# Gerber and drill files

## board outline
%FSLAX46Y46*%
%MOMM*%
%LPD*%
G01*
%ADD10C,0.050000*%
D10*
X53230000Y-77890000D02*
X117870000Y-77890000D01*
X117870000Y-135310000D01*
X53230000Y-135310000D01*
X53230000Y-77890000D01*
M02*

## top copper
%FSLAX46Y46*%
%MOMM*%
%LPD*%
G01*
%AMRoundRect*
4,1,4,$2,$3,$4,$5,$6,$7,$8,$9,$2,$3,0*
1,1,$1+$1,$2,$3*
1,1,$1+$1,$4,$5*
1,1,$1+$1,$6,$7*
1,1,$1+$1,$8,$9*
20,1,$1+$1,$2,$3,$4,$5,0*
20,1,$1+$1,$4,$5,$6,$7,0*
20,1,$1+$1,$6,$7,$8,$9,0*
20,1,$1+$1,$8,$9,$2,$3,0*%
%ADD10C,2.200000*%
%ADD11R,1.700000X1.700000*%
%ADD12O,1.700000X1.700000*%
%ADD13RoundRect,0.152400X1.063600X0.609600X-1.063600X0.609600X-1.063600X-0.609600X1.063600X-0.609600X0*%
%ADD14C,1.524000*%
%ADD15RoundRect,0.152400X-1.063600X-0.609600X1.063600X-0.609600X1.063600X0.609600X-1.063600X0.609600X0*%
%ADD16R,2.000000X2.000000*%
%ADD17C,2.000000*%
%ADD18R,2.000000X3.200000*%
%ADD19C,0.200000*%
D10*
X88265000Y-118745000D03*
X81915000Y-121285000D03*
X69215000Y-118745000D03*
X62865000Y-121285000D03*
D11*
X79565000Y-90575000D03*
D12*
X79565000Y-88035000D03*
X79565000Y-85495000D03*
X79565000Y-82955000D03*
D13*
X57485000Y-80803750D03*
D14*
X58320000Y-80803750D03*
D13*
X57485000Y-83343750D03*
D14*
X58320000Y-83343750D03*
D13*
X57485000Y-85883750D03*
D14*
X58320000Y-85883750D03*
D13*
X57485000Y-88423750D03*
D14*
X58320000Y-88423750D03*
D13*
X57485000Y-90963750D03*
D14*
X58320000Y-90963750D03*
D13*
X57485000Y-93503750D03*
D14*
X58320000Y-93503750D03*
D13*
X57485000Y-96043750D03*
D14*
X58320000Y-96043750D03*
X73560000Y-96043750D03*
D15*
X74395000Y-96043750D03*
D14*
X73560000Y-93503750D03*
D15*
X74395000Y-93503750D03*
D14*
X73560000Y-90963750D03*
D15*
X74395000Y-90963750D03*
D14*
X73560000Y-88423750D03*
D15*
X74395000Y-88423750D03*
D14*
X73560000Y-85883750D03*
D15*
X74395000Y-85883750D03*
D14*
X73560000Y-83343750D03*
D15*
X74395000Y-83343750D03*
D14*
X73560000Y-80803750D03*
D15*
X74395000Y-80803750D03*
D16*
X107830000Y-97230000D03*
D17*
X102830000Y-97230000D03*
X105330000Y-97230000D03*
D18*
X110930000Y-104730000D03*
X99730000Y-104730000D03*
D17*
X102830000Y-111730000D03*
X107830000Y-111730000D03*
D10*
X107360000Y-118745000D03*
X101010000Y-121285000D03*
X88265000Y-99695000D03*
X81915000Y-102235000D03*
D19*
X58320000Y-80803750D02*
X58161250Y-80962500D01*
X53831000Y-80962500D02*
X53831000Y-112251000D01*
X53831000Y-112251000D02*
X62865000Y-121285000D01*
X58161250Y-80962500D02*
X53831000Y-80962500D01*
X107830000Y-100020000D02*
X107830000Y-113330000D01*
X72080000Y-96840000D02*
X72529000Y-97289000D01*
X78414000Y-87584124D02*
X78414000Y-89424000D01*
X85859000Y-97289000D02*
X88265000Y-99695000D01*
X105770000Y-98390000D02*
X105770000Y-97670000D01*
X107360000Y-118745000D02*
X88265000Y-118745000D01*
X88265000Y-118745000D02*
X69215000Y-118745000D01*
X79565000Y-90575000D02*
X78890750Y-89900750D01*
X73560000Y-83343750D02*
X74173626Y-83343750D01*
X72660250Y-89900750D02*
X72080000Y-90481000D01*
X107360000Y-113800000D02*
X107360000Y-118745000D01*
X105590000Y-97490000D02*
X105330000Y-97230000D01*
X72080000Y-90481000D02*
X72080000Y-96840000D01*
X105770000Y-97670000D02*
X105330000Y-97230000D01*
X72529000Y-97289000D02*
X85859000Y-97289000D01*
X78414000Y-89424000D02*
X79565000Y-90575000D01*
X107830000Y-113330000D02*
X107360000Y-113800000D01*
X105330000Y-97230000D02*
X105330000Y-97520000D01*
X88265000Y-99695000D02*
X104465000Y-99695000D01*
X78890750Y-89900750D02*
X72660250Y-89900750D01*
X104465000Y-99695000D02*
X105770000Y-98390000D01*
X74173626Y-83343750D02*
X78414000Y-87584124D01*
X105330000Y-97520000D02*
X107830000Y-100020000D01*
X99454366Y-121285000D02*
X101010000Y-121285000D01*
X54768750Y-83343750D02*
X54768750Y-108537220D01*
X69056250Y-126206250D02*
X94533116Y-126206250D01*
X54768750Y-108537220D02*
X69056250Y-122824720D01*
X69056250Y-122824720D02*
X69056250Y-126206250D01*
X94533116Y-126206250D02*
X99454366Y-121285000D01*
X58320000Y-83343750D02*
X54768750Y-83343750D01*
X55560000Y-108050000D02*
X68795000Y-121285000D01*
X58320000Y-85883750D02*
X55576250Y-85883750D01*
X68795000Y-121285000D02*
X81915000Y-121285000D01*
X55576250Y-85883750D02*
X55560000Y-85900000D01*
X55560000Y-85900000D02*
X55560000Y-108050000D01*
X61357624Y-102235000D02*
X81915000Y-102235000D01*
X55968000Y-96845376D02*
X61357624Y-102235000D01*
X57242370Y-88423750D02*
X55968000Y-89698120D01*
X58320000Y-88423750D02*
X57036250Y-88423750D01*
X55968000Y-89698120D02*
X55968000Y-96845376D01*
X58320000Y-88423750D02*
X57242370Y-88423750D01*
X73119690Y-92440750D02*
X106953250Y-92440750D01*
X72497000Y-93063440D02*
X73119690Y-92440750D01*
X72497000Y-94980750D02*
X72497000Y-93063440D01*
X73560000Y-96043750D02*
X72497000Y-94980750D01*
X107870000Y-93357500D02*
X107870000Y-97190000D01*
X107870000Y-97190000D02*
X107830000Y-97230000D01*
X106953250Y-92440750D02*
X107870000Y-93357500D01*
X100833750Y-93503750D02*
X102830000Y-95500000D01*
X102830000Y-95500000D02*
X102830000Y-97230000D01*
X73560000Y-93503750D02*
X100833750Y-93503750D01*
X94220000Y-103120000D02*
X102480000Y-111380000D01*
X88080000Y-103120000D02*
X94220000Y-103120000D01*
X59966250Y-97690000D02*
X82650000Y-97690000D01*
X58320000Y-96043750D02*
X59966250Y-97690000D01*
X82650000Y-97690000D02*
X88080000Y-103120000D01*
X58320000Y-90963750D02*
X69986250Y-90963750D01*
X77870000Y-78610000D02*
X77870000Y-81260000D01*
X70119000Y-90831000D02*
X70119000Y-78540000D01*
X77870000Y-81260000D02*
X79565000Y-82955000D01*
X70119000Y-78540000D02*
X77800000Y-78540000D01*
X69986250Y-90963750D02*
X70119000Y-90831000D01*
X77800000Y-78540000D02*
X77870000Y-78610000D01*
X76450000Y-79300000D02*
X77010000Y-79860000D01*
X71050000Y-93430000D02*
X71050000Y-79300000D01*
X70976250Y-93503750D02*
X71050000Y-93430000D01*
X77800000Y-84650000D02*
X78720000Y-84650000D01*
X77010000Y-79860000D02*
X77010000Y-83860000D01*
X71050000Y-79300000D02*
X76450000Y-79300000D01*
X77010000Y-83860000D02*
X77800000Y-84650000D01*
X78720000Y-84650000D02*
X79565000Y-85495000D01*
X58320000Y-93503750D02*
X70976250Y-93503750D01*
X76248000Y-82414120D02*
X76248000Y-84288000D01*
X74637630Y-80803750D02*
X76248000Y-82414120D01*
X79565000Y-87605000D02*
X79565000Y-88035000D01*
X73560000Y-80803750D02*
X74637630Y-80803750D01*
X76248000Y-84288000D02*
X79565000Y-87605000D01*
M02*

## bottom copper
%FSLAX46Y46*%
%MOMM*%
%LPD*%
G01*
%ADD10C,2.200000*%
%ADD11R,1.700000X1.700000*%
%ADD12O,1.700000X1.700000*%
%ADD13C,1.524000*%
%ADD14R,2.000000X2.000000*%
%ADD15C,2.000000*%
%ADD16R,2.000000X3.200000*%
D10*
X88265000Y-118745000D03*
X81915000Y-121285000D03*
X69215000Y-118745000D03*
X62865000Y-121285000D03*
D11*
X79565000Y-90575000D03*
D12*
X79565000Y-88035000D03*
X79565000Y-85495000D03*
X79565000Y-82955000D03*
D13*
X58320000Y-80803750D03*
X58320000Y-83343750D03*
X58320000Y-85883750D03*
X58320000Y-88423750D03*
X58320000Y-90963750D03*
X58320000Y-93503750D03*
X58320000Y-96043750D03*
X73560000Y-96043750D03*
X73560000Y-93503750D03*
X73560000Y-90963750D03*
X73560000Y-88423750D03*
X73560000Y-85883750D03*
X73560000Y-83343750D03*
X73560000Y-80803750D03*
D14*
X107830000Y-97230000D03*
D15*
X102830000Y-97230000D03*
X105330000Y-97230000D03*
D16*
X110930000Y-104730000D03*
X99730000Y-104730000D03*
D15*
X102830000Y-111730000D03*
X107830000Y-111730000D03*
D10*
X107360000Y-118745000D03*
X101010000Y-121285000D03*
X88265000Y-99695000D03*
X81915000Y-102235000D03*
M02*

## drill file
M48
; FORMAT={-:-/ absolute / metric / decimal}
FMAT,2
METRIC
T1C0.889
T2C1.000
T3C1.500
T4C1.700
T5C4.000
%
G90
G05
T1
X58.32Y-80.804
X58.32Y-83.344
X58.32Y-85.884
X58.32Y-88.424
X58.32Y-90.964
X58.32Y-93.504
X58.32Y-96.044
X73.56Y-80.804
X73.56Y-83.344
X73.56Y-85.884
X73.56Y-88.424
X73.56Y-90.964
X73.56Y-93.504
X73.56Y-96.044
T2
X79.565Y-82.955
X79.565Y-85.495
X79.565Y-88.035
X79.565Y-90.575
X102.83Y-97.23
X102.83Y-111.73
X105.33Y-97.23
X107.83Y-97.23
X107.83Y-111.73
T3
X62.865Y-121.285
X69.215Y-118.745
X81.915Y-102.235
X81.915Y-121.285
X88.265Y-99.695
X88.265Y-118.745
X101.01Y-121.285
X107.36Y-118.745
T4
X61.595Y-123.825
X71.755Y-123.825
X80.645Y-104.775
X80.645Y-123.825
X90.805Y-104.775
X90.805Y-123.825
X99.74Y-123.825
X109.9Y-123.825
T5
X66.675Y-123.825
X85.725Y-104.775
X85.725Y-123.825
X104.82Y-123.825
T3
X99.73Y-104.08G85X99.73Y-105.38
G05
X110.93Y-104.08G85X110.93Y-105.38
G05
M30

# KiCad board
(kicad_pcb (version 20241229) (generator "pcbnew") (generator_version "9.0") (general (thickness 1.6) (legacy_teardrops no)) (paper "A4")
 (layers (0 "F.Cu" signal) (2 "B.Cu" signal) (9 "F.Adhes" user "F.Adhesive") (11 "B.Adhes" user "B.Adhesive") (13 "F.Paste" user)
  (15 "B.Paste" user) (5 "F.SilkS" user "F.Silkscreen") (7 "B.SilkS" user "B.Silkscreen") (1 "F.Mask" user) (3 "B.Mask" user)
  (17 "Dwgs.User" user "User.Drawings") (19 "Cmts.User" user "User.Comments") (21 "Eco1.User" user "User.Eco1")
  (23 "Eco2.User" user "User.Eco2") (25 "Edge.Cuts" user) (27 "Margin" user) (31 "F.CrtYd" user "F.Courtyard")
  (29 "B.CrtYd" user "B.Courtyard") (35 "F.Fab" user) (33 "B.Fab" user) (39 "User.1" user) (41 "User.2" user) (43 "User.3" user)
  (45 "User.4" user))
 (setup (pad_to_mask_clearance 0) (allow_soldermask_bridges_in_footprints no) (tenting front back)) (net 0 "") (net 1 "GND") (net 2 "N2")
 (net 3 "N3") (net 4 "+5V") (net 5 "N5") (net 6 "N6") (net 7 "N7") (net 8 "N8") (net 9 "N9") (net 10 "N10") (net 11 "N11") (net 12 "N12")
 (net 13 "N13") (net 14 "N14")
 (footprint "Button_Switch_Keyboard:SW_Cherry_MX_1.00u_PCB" (layer "F.Cu") (at 88.265 118.745)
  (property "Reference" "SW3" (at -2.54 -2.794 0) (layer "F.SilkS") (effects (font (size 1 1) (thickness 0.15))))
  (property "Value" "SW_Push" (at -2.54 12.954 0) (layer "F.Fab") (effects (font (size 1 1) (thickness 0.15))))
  (pad "" np_thru_hole circle (at -7.62 5.08) (size 1.7 1.7) (drill 1.7) (layers "*.Cu" "*.Mask"))
  (pad "" np_thru_hole circle (at -2.54 5.08) (size 4 4) (drill 4) (layers "*.Cu" "*.Mask"))
  (pad "" np_thru_hole circle (at 2.54 5.08) (size 1.7 1.7) (drill 1.7) (layers "*.Cu" "*.Mask"))
  (pad "1" thru_hole circle (at 0 0) (size 2.2 2.2) (drill 1.5) (layers "*.Cu" "*.Mask") (remove_unused_layers no) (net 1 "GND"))
  (pad "2" thru_hole circle (at -6.35 2.54) (size 2.2 2.2) (drill 1.5) (layers "*.Cu" "*.Mask") (remove_unused_layers no) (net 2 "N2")))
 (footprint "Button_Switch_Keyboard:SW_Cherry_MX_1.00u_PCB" (layer "F.Cu") (at 69.215 118.745)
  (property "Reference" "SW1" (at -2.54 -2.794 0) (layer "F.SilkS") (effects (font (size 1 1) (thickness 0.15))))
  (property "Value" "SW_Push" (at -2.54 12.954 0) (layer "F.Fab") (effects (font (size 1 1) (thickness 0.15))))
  (pad "" np_thru_hole circle (at -7.62 5.08) (size 1.7 1.7) (drill 1.7) (layers "*.Cu" "*.Mask"))
  (pad "" np_thru_hole circle (at -2.54 5.08) (size 4 4) (drill 4) (layers "*.Cu" "*.Mask"))
  (pad "" np_thru_hole circle (at 2.54 5.08) (size 1.7 1.7) (drill 1.7) (layers "*.Cu" "*.Mask"))
  (pad "1" thru_hole circle (at 0 0) (size 2.2 2.2) (drill 1.5) (layers "*.Cu" "*.Mask") (remove_unused_layers no) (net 1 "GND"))
  (pad "2" thru_hole circle (at -6.35 2.54) (size 2.2 2.2) (drill 1.5) (layers "*.Cu" "*.Mask") (remove_unused_layers no) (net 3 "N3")))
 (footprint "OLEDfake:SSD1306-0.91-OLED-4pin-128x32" (layer "F.Cu") (at 116.065 92.765 180)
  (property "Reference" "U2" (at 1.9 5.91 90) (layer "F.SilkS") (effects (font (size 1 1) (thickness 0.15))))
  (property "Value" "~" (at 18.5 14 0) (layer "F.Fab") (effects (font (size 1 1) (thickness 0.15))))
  (pad "1" thru_hole rect (at 36.5 2.19 180) (size 1.7 1.7) (drill 1) (layers "*.Cu" "*.Mask") (remove_unused_layers no) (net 1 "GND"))
  (pad "2" thru_hole oval (at 36.5 4.73 180) (size 1.7 1.7) (drill 1) (layers "*.Cu" "*.Mask") (remove_unused_layers no) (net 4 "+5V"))
  (pad "3" thru_hole oval (at 36.5 7.27 180) (size 1.7 1.7) (drill 1) (layers "*.Cu" "*.Mask") (remove_unused_layers no) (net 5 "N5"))
  (pad "4" thru_hole oval (at 36.5 9.81 180) (size 1.7 1.7) (drill 1) (layers "*.Cu" "*.Mask") (remove_unused_layers no) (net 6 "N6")))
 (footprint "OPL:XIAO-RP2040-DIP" (layer "F.Cu") (at 65.94 88.42375)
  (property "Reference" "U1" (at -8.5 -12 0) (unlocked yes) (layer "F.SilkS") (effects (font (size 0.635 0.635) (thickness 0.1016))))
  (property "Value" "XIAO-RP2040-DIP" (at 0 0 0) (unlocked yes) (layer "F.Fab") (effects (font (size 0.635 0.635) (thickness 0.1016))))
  (pad "1" smd roundrect (at -8.455 -7.62 180) (size 2.432 1.524) (layers "F.Cu" "F.Mask") (roundrect_rratio 0.1) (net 3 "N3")
   (thermal_bridge_angle 45))
  (pad "1" thru_hole circle (at -7.62 -7.62 180) (size 1.524 1.524) (drill 0.889) (layers "*.Cu" "*.Mask") (remove_unused_layers no)
   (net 3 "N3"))
  (pad "2" smd roundrect (at -8.455 -5.08 180) (size 2.432 1.524) (layers "F.Cu" "F.Mask") (roundrect_rratio 0.1) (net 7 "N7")
   (thermal_bridge_angle 45))
  (pad "2" thru_hole circle (at -7.62 -5.08 180) (size 1.524 1.524) (drill 0.889) (layers "*.Cu" "*.Mask") (remove_unused_layers no)
   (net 7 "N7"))
  (pad "3" smd roundrect (at -8.455 -2.54 180) (size 2.432 1.524) (layers "F.Cu" "F.Mask") (roundrect_rratio 0.1) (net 2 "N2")
   (thermal_bridge_angle 45))
  (pad "3" thru_hole circle (at -7.62 -2.54 180) (size 1.524 1.524) (drill 0.889) (layers "*.Cu" "*.Mask") (remove_unused_layers no)
   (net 2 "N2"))
  (pad "4" smd roundrect (at -8.455 0 180) (size 2.432 1.524) (layers "F.Cu" "F.Mask") (roundrect_rratio 0.1) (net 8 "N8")
   (thermal_bridge_angle 45))
  (pad "4" thru_hole circle (at -7.62 0 180) (size 1.524 1.524) (drill 0.889) (layers "*.Cu" "*.Mask") (remove_unused_layers no)
   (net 8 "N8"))
  (pad "5" smd roundrect (at -8.455 2.54 180) (size 2.432 1.524) (layers "F.Cu" "F.Mask") (roundrect_rratio 0.1) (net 6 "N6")
   (thermal_bridge_angle 45))
  (pad "5" thru_hole circle (at -7.62 2.54 180) (size 1.524 1.524) (drill 0.889) (layers "*.Cu" "*.Mask") (remove_unused_layers no)
   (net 6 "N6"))
  (pad "6" smd roundrect (at -8.455 5.08 180) (size 2.432 1.524) (layers "F.Cu" "F.Mask") (roundrect_rratio 0.1) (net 5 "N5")
   (thermal_bridge_angle 45))
  (pad "6" thru_hole circle (at -7.62 5.08 180) (size 1.524 1.524) (drill 0.889) (layers "*.Cu" "*.Mask") (remove_unused_layers no)
   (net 5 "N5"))
  (pad "7" smd roundrect (at -8.455 7.62 180) (size 2.432 1.524) (layers "F.Cu" "F.Mask") (roundrect_rratio 0.1) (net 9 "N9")
   (thermal_bridge_angle 45))
  (pad "7" thru_hole circle (at -7.62 7.62 180) (size 1.524 1.524) (drill 0.889) (layers "*.Cu" "*.Mask") (remove_unused_layers no)
   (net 9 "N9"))
  (pad "8" thru_hole circle (at 7.62 7.62) (size 1.524 1.524) (drill 0.889) (layers "*.Cu" "*.Mask") (remove_unused_layers no)
   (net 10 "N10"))
  (pad "8" smd roundrect (at 8.455 7.62) (size 2.432 1.524) (layers "F.Cu" "F.Mask") (roundrect_rratio 0.1) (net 10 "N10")
   (thermal_bridge_angle 45))
  (pad "9" thru_hole circle (at 7.62 5.08) (size 1.524 1.524) (drill 0.889) (layers "*.Cu" "*.Mask") (remove_unused_layers no)
   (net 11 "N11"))
  (pad "9" smd roundrect (at 8.455 5.08) (size 2.432 1.524) (layers "F.Cu" "F.Mask") (roundrect_rratio 0.1) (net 11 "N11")
   (thermal_bridge_angle 45))
  (pad "10" thru_hole circle (at 7.62 2.54) (size 1.524 1.524) (drill 0.889) (layers "*.Cu" "*.Mask") (remove_unused_layers no)
   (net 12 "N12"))
  (pad "10" smd roundrect (at 8.455 2.54) (size 2.432 1.524) (layers "F.Cu" "F.Mask") (roundrect_rratio 0.1) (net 12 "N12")
   (thermal_bridge_angle 45))
  (pad "11" thru_hole circle (at 7.62 0) (size 1.524 1.524) (drill 0.889) (layers "*.Cu" "*.Mask") (remove_unused_layers no) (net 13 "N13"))
  (pad "11" smd roundrect (at 8.455 0) (size 2.432 1.524) (layers "F.Cu" "F.Mask") (roundrect_rratio 0.1) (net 13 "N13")
   (thermal_bridge_angle 45))
  (pad "12" thru_hole circle (at 7.62 -2.54) (size 1.524 1.524) (drill 0.889) (layers "*.Cu" "*.Mask") (remove_unused_layers no)
   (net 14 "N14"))
  (pad "12" smd roundrect (at 8.455 -2.54) (size 2.432 1.524) (layers "F.Cu" "F.Mask") (roundrect_rratio 0.1) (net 14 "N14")
   (thermal_bridge_angle 45))
  (pad "13" thru_hole circle (at 7.62 -5.08) (size 1.524 1.524) (drill 0.889) (layers "*.Cu" "*.Mask") (remove_unused_layers no)
   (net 1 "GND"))
  (pad "13" smd roundrect (at 8.455 -5.08) (size 2.432 1.524) (layers "F.Cu" "F.Mask") (roundrect_rratio 0.1) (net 1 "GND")
   (thermal_bridge_angle 45))
  (pad "14" thru_hole circle (at 7.62 -7.62) (size 1.524 1.524) (drill 0.889) (layers "*.Cu" "*.Mask") (remove_unused_layers no)
   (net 4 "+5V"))
  (pad "14" smd roundrect (at 8.455 -7.62) (size 2.432 1.524) (layers "F.Cu" "F.Mask") (roundrect_rratio 0.1) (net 4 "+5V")
   (thermal_bridge_angle 45)))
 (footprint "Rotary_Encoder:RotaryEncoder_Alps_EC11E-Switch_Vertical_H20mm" (layer "F.Cu") (at 107.83 97.23 -90)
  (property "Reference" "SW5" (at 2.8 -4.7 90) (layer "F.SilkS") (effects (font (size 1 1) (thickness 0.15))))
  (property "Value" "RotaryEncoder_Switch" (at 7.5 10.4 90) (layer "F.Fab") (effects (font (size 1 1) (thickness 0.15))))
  (pad "A" thru_hole rect (at 0 0 270) (size 2 2) (drill 1) (layers "*.Cu" "*.Mask") (remove_unused_layers no) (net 10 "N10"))
  (pad "B" thru_hole circle (at 0 5 270) (size 2 2) (drill 1) (layers "*.Cu" "*.Mask") (remove_unused_layers no) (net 11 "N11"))
  (pad "C" thru_hole circle (at 0 2.5 270) (size 2 2) (drill 1) (layers "*.Cu" "*.Mask") (remove_unused_layers no) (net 1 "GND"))
  (pad "MP" thru_hole rect (at 7.5 -3.1 270) (size 3.2 2) (drill oval 2.8 1.5) (layers "*.Cu" "*.Mask") (remove_unused_layers no))
  (pad "MP" thru_hole rect (at 7.5 8.1 270) (size 3.2 2) (drill oval 2.8 1.5) (layers "*.Cu" "*.Mask") (remove_unused_layers no))
  (pad "S1" thru_hole circle (at 14.5 5 270) (size 2 2) (drill 1) (layers "*.Cu" "*.Mask") (remove_unused_layers no) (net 9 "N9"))
  (pad "S2" thru_hole circle (at 14.5 0 270) (size 2 2) (drill 1) (layers "*.Cu" "*.Mask") (remove_unused_layers no) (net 1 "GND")))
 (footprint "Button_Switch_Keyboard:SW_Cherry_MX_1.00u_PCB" (layer "F.Cu") (at 107.36 118.745)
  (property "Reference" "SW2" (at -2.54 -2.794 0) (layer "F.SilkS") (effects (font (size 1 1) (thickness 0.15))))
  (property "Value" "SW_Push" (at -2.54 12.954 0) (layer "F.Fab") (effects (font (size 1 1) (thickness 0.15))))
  (pad "" np_thru_hole circle (at -7.62 5.08) (size 1.7 1.7) (drill 1.7) (layers "*.Cu" "*.Mask"))
  (pad "" np_thru_hole circle (at -2.54 5.08) (size 4 4) (drill 4) (layers "*.Cu" "*.Mask"))
  (pad "" np_thru_hole circle (at 2.54 5.08) (size 1.7 1.7) (drill 1.7) (layers "*.Cu" "*.Mask"))
  (pad "1" thru_hole circle (at 0 0) (size 2.2 2.2) (drill 1.5) (layers "*.Cu" "*.Mask") (remove_unused_layers no) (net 1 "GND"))
  (pad "2" thru_hole circle (at -6.35 2.54) (size 2.2 2.2) (drill 1.5) (layers "*.Cu" "*.Mask") (remove_unused_layers no) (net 7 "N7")))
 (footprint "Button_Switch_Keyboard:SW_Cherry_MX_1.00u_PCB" (layer "F.Cu") (at 88.265 99.695)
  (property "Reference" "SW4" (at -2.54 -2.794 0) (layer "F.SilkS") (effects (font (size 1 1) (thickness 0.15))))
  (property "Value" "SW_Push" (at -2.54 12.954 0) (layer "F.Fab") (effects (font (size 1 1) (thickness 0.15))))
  (pad "" np_thru_hole circle (at -7.62 5.08) (size 1.7 1.7) (drill 1.7) (layers "*.Cu" "*.Mask"))
  (pad "" np_thru_hole circle (at -2.54 5.08) (size 4 4) (drill 4) (layers "*.Cu" "*.Mask"))
  (pad "" np_thru_hole circle (at 2.54 5.08) (size 1.7 1.7) (drill 1.7) (layers "*.Cu" "*.Mask"))
  (pad "1" thru_hole circle (at 0 0) (size 2.2 2.2) (drill 1.5) (layers "*.Cu" "*.Mask") (remove_unused_layers no) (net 1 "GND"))
  (pad "2" thru_hole circle (at -6.35 2.54) (size 2.2 2.2) (drill 1.5) (layers "*.Cu" "*.Mask") (remove_unused_layers no) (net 8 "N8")))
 (gr_rect (start 53.23 77.89) (end 117.87 135.31) (stroke (width 0.05) (type default)) (fill no) (layer "Edge.Cuts"))
 (segment (start 58.32 80.80375) (end 58.16125 80.9625) (width 0.2) (layer "F.Cu") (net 3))
 (segment (start 53.831 80.9625) (end 53.831 112.251) (width 0.2) (layer "F.Cu") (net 3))
 (segment (start 53.831 112.251) (end 62.865 121.285) (width 0.2) (layer "F.Cu") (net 3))
 (segment (start 58.16125 80.9625) (end 53.831 80.9625) (width 0.2) (layer "F.Cu") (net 3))
 (segment (start 107.83 100.02) (end 107.83 113.33) (width 0.2) (layer "F.Cu") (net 1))
 (segment (start 72.08 96.84) (end 72.529 97.289) (width 0.2) (layer "F.Cu") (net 1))
 (segment (start 78.414 87.584124) (end 78.414 89.424) (width 0.2) (layer "F.Cu") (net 1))
 (segment (start 85.859 97.289) (end 88.265 99.695) (width 0.2) (layer "F.Cu") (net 1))
 (segment (start 105.77 98.39) (end 105.77 97.67) (width 0.2) (layer "F.Cu") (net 1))
 (segment (start 107.36 118.745) (end 88.265 118.745) (width 0.2) (layer "F.Cu") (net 1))
 (segment (start 88.265 118.745) (end 69.215 118.745) (width 0.2) (layer "F.Cu") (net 1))
 (segment (start 79.565 90.575) (end 78.89075 89.90075) (width 0.2) (layer "F.Cu") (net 1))
 (segment (start 73.56 83.34375) (end 74.173626 83.34375) (width 0.2) (layer "F.Cu") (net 1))
 (segment (start 72.66025 89.90075) (end 72.08 90.481) (width 0.2) (layer "F.Cu") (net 1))
 (segment (start 107.36 113.8) (end 107.36 118.745) (width 0.2) (layer "F.Cu") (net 1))
 (segment (start 105.59 97.49) (end 105.33 97.23) (width 0.2) (layer "F.Cu") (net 1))
 (segment (start 72.08 90.481) (end 72.08 96.84) (width 0.2) (layer "F.Cu") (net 1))
 (segment (start 105.77 97.67) (end 105.33 97.23) (width 0.2) (layer "F.Cu") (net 1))
 (segment (start 72.529 97.289) (end 85.859 97.289) (width 0.2) (layer "F.Cu") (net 1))
 (segment (start 78.414 89.424) (end 79.565 90.575) (width 0.2) (layer "F.Cu") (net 1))
 (segment (start 107.83 113.33) (end 107.36 113.8) (width 0.2) (layer "F.Cu") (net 1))
 (segment (start 105.33 97.23) (end 105.33 97.52) (width 0.2) (layer "F.Cu") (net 1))
 (segment (start 88.265 99.695) (end 104.465 99.695) (width 0.2) (layer "F.Cu") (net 1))
 (segment (start 78.89075 89.90075) (end 72.66025 89.90075) (width 0.2) (layer "F.Cu") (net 1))
 (segment (start 104.465 99.695) (end 105.77 98.39) (width 0.2) (layer "F.Cu") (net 1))
 (segment (start 74.173626 83.34375) (end 78.414 87.584124) (width 0.2) (layer "F.Cu") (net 1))
 (segment (start 105.33 97.52) (end 107.83 100.02) (width 0.2) (layer "F.Cu") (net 1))
 (segment (start 99.454366 121.285) (end 101.01 121.285) (width 0.2) (layer "F.Cu") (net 7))
 (segment (start 54.76875 83.34375) (end 54.76875 108.53722) (width 0.2) (layer "F.Cu") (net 7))
 (segment (start 69.05625 126.20625) (end 94.533116 126.20625) (width 0.2) (layer "F.Cu") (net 7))
 (segment (start 54.76875 108.53722) (end 69.05625 122.82472) (width 0.2) (layer "F.Cu") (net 7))
 (segment (start 69.05625 122.82472) (end 69.05625 126.20625) (width 0.2) (layer "F.Cu") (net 7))
 (segment (start 94.533116 126.20625) (end 99.454366 121.285) (width 0.2) (layer "F.Cu") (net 7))
 (segment (start 58.32 83.34375) (end 54.76875 83.34375) (width 0.2) (layer "F.Cu") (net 7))
 (segment (start 55.56 108.05) (end 68.795 121.285) (width 0.2) (layer "F.Cu") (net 2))
 (segment (start 58.32 85.88375) (end 55.57625 85.88375) (width 0.2) (layer "F.Cu") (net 2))
 (segment (start 68.795 121.285) (end 81.915 121.285) (width 0.2) (layer "F.Cu") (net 2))
 (segment (start 55.57625 85.88375) (end 55.56 85.9) (width 0.2) (layer "F.Cu") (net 2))
 (segment (start 55.56 85.9) (end 55.56 108.05) (width 0.2) (layer "F.Cu") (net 2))
 (segment (start 61.357624 102.235) (end 81.915 102.235) (width 0.2) (layer "F.Cu") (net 8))
 (segment (start 55.968 96.845376) (end 61.357624 102.235) (width 0.2) (layer "F.Cu") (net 8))
 (segment (start 57.24237 88.42375) (end 55.968 89.69812) (width 0.2) (layer "F.Cu") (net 8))
 (segment (start 58.32 88.42375) (end 57.03625 88.42375) (width 0.2) (layer "F.Cu") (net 8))
 (segment (start 55.968 89.69812) (end 55.968 96.845376) (width 0.2) (layer "F.Cu") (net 8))
 (segment (start 58.32 88.42375) (end 57.24237 88.42375) (width 0.2) (layer "F.Cu") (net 8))
 (segment (start 73.11969 92.44075) (end 106.95325 92.44075) (width 0.2) (layer "F.Cu") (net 10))
 (segment (start 72.497 93.06344) (end 73.11969 92.44075) (width 0.2) (layer "F.Cu") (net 10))
 (segment (start 72.497 94.98075) (end 72.497 93.06344) (width 0.2) (layer "F.Cu") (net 10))
 (segment (start 73.56 96.04375) (end 72.497 94.98075) (width 0.2) (layer "F.Cu") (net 10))
 (segment (start 107.87 93.3575) (end 107.87 97.19) (width 0.2) (layer "F.Cu") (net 10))
 (segment (start 107.87 97.19) (end 107.83 97.23) (width 0.2) (layer "F.Cu") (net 10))
 (segment (start 106.95325 92.44075) (end 107.87 93.3575) (width 0.2) (layer "F.Cu") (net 10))
 (segment (start 100.83375 93.50375) (end 102.83 95.5) (width 0.2) (layer "F.Cu") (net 11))
 (segment (start 102.83 95.5) (end 102.83 97.23) (width 0.2) (layer "F.Cu") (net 11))
 (segment (start 73.56 93.50375) (end 100.83375 93.50375) (width 0.2) (layer "F.Cu") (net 11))
 (segment (start 94.22 103.12) (end 102.48 111.38) (width 0.2) (layer "F.Cu") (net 9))
 (segment (start 88.08 103.12) (end 94.22 103.12) (width 0.2) (layer "F.Cu") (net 9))
 (segment (start 59.96625 97.69) (end 82.65 97.69) (width 0.2) (layer "F.Cu") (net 9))
 (segment (start 58.32 96.04375) (end 59.96625 97.69) (width 0.2) (layer "F.Cu") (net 9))
 (segment (start 82.65 97.69) (end 88.08 103.12) (width 0.2) (layer "F.Cu") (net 9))
 (segment (start 58.32 90.96375) (end 69.98625 90.96375) (width 0.2) (layer "F.Cu") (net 6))
 (segment (start 77.87 78.61) (end 77.87 81.26) (width 0.2) (layer "F.Cu") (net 6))
 (segment (start 70.119 90.831) (end 70.119 78.54) (width 0.2) (layer "F.Cu") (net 6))
 (segment (start 77.87 81.26) (end 79.565 82.955) (width 0.2) (layer "F.Cu") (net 6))
 (segment (start 70.119 78.54) (end 77.8 78.54) (width 0.2) (layer "F.Cu") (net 6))
 (segment (start 69.98625 90.96375) (end 70.119 90.831) (width 0.2) (layer "F.Cu") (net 6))
 (segment (start 77.8 78.54) (end 77.87 78.61) (width 0.2) (layer "F.Cu") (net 6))
 (segment (start 76.45 79.3) (end 77.01 79.86) (width 0.2) (layer "F.Cu") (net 5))
 (segment (start 71.05 93.43) (end 71.05 79.3) (width 0.2) (layer "F.Cu") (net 5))
 (segment (start 70.97625 93.50375) (end 71.05 93.43) (width 0.2) (layer "F.Cu") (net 5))
 (segment (start 77.8 84.65) (end 78.72 84.65) (width 0.2) (layer "F.Cu") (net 5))
 (segment (start 77.01 79.86) (end 77.01 83.86) (width 0.2) (layer "F.Cu") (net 5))
 (segment (start 71.05 79.3) (end 76.45 79.3) (width 0.2) (layer "F.Cu") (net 5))
 (segment (start 77.01 83.86) (end 77.8 84.65) (width 0.2) (layer "F.Cu") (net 5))
 (segment (start 78.72 84.65) (end 79.565 85.495) (width 0.2) (layer "F.Cu") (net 5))
 (segment (start 58.32 93.50375) (end 70.97625 93.50375) (width 0.2) (layer "F.Cu") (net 5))
 (segment (start 76.248 82.41412) (end 76.248 84.288) (width 0.2) (layer "F.Cu") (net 4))
 (segment (start 74.63763 80.80375) (end 76.248 82.41412) (width 0.2) (layer "F.Cu") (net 4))
 (segment (start 79.565 87.605) (end 79.565 88.035) (width 0.2) (layer "F.Cu") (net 4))
 (segment (start 73.56 80.80375) (end 74.63763 80.80375) (width 0.2) (layer "F.Cu") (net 4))
 (segment (start 76.248 84.288) (end 79.565 87.605) (width 0.2) (layer "F.Cu") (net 4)))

